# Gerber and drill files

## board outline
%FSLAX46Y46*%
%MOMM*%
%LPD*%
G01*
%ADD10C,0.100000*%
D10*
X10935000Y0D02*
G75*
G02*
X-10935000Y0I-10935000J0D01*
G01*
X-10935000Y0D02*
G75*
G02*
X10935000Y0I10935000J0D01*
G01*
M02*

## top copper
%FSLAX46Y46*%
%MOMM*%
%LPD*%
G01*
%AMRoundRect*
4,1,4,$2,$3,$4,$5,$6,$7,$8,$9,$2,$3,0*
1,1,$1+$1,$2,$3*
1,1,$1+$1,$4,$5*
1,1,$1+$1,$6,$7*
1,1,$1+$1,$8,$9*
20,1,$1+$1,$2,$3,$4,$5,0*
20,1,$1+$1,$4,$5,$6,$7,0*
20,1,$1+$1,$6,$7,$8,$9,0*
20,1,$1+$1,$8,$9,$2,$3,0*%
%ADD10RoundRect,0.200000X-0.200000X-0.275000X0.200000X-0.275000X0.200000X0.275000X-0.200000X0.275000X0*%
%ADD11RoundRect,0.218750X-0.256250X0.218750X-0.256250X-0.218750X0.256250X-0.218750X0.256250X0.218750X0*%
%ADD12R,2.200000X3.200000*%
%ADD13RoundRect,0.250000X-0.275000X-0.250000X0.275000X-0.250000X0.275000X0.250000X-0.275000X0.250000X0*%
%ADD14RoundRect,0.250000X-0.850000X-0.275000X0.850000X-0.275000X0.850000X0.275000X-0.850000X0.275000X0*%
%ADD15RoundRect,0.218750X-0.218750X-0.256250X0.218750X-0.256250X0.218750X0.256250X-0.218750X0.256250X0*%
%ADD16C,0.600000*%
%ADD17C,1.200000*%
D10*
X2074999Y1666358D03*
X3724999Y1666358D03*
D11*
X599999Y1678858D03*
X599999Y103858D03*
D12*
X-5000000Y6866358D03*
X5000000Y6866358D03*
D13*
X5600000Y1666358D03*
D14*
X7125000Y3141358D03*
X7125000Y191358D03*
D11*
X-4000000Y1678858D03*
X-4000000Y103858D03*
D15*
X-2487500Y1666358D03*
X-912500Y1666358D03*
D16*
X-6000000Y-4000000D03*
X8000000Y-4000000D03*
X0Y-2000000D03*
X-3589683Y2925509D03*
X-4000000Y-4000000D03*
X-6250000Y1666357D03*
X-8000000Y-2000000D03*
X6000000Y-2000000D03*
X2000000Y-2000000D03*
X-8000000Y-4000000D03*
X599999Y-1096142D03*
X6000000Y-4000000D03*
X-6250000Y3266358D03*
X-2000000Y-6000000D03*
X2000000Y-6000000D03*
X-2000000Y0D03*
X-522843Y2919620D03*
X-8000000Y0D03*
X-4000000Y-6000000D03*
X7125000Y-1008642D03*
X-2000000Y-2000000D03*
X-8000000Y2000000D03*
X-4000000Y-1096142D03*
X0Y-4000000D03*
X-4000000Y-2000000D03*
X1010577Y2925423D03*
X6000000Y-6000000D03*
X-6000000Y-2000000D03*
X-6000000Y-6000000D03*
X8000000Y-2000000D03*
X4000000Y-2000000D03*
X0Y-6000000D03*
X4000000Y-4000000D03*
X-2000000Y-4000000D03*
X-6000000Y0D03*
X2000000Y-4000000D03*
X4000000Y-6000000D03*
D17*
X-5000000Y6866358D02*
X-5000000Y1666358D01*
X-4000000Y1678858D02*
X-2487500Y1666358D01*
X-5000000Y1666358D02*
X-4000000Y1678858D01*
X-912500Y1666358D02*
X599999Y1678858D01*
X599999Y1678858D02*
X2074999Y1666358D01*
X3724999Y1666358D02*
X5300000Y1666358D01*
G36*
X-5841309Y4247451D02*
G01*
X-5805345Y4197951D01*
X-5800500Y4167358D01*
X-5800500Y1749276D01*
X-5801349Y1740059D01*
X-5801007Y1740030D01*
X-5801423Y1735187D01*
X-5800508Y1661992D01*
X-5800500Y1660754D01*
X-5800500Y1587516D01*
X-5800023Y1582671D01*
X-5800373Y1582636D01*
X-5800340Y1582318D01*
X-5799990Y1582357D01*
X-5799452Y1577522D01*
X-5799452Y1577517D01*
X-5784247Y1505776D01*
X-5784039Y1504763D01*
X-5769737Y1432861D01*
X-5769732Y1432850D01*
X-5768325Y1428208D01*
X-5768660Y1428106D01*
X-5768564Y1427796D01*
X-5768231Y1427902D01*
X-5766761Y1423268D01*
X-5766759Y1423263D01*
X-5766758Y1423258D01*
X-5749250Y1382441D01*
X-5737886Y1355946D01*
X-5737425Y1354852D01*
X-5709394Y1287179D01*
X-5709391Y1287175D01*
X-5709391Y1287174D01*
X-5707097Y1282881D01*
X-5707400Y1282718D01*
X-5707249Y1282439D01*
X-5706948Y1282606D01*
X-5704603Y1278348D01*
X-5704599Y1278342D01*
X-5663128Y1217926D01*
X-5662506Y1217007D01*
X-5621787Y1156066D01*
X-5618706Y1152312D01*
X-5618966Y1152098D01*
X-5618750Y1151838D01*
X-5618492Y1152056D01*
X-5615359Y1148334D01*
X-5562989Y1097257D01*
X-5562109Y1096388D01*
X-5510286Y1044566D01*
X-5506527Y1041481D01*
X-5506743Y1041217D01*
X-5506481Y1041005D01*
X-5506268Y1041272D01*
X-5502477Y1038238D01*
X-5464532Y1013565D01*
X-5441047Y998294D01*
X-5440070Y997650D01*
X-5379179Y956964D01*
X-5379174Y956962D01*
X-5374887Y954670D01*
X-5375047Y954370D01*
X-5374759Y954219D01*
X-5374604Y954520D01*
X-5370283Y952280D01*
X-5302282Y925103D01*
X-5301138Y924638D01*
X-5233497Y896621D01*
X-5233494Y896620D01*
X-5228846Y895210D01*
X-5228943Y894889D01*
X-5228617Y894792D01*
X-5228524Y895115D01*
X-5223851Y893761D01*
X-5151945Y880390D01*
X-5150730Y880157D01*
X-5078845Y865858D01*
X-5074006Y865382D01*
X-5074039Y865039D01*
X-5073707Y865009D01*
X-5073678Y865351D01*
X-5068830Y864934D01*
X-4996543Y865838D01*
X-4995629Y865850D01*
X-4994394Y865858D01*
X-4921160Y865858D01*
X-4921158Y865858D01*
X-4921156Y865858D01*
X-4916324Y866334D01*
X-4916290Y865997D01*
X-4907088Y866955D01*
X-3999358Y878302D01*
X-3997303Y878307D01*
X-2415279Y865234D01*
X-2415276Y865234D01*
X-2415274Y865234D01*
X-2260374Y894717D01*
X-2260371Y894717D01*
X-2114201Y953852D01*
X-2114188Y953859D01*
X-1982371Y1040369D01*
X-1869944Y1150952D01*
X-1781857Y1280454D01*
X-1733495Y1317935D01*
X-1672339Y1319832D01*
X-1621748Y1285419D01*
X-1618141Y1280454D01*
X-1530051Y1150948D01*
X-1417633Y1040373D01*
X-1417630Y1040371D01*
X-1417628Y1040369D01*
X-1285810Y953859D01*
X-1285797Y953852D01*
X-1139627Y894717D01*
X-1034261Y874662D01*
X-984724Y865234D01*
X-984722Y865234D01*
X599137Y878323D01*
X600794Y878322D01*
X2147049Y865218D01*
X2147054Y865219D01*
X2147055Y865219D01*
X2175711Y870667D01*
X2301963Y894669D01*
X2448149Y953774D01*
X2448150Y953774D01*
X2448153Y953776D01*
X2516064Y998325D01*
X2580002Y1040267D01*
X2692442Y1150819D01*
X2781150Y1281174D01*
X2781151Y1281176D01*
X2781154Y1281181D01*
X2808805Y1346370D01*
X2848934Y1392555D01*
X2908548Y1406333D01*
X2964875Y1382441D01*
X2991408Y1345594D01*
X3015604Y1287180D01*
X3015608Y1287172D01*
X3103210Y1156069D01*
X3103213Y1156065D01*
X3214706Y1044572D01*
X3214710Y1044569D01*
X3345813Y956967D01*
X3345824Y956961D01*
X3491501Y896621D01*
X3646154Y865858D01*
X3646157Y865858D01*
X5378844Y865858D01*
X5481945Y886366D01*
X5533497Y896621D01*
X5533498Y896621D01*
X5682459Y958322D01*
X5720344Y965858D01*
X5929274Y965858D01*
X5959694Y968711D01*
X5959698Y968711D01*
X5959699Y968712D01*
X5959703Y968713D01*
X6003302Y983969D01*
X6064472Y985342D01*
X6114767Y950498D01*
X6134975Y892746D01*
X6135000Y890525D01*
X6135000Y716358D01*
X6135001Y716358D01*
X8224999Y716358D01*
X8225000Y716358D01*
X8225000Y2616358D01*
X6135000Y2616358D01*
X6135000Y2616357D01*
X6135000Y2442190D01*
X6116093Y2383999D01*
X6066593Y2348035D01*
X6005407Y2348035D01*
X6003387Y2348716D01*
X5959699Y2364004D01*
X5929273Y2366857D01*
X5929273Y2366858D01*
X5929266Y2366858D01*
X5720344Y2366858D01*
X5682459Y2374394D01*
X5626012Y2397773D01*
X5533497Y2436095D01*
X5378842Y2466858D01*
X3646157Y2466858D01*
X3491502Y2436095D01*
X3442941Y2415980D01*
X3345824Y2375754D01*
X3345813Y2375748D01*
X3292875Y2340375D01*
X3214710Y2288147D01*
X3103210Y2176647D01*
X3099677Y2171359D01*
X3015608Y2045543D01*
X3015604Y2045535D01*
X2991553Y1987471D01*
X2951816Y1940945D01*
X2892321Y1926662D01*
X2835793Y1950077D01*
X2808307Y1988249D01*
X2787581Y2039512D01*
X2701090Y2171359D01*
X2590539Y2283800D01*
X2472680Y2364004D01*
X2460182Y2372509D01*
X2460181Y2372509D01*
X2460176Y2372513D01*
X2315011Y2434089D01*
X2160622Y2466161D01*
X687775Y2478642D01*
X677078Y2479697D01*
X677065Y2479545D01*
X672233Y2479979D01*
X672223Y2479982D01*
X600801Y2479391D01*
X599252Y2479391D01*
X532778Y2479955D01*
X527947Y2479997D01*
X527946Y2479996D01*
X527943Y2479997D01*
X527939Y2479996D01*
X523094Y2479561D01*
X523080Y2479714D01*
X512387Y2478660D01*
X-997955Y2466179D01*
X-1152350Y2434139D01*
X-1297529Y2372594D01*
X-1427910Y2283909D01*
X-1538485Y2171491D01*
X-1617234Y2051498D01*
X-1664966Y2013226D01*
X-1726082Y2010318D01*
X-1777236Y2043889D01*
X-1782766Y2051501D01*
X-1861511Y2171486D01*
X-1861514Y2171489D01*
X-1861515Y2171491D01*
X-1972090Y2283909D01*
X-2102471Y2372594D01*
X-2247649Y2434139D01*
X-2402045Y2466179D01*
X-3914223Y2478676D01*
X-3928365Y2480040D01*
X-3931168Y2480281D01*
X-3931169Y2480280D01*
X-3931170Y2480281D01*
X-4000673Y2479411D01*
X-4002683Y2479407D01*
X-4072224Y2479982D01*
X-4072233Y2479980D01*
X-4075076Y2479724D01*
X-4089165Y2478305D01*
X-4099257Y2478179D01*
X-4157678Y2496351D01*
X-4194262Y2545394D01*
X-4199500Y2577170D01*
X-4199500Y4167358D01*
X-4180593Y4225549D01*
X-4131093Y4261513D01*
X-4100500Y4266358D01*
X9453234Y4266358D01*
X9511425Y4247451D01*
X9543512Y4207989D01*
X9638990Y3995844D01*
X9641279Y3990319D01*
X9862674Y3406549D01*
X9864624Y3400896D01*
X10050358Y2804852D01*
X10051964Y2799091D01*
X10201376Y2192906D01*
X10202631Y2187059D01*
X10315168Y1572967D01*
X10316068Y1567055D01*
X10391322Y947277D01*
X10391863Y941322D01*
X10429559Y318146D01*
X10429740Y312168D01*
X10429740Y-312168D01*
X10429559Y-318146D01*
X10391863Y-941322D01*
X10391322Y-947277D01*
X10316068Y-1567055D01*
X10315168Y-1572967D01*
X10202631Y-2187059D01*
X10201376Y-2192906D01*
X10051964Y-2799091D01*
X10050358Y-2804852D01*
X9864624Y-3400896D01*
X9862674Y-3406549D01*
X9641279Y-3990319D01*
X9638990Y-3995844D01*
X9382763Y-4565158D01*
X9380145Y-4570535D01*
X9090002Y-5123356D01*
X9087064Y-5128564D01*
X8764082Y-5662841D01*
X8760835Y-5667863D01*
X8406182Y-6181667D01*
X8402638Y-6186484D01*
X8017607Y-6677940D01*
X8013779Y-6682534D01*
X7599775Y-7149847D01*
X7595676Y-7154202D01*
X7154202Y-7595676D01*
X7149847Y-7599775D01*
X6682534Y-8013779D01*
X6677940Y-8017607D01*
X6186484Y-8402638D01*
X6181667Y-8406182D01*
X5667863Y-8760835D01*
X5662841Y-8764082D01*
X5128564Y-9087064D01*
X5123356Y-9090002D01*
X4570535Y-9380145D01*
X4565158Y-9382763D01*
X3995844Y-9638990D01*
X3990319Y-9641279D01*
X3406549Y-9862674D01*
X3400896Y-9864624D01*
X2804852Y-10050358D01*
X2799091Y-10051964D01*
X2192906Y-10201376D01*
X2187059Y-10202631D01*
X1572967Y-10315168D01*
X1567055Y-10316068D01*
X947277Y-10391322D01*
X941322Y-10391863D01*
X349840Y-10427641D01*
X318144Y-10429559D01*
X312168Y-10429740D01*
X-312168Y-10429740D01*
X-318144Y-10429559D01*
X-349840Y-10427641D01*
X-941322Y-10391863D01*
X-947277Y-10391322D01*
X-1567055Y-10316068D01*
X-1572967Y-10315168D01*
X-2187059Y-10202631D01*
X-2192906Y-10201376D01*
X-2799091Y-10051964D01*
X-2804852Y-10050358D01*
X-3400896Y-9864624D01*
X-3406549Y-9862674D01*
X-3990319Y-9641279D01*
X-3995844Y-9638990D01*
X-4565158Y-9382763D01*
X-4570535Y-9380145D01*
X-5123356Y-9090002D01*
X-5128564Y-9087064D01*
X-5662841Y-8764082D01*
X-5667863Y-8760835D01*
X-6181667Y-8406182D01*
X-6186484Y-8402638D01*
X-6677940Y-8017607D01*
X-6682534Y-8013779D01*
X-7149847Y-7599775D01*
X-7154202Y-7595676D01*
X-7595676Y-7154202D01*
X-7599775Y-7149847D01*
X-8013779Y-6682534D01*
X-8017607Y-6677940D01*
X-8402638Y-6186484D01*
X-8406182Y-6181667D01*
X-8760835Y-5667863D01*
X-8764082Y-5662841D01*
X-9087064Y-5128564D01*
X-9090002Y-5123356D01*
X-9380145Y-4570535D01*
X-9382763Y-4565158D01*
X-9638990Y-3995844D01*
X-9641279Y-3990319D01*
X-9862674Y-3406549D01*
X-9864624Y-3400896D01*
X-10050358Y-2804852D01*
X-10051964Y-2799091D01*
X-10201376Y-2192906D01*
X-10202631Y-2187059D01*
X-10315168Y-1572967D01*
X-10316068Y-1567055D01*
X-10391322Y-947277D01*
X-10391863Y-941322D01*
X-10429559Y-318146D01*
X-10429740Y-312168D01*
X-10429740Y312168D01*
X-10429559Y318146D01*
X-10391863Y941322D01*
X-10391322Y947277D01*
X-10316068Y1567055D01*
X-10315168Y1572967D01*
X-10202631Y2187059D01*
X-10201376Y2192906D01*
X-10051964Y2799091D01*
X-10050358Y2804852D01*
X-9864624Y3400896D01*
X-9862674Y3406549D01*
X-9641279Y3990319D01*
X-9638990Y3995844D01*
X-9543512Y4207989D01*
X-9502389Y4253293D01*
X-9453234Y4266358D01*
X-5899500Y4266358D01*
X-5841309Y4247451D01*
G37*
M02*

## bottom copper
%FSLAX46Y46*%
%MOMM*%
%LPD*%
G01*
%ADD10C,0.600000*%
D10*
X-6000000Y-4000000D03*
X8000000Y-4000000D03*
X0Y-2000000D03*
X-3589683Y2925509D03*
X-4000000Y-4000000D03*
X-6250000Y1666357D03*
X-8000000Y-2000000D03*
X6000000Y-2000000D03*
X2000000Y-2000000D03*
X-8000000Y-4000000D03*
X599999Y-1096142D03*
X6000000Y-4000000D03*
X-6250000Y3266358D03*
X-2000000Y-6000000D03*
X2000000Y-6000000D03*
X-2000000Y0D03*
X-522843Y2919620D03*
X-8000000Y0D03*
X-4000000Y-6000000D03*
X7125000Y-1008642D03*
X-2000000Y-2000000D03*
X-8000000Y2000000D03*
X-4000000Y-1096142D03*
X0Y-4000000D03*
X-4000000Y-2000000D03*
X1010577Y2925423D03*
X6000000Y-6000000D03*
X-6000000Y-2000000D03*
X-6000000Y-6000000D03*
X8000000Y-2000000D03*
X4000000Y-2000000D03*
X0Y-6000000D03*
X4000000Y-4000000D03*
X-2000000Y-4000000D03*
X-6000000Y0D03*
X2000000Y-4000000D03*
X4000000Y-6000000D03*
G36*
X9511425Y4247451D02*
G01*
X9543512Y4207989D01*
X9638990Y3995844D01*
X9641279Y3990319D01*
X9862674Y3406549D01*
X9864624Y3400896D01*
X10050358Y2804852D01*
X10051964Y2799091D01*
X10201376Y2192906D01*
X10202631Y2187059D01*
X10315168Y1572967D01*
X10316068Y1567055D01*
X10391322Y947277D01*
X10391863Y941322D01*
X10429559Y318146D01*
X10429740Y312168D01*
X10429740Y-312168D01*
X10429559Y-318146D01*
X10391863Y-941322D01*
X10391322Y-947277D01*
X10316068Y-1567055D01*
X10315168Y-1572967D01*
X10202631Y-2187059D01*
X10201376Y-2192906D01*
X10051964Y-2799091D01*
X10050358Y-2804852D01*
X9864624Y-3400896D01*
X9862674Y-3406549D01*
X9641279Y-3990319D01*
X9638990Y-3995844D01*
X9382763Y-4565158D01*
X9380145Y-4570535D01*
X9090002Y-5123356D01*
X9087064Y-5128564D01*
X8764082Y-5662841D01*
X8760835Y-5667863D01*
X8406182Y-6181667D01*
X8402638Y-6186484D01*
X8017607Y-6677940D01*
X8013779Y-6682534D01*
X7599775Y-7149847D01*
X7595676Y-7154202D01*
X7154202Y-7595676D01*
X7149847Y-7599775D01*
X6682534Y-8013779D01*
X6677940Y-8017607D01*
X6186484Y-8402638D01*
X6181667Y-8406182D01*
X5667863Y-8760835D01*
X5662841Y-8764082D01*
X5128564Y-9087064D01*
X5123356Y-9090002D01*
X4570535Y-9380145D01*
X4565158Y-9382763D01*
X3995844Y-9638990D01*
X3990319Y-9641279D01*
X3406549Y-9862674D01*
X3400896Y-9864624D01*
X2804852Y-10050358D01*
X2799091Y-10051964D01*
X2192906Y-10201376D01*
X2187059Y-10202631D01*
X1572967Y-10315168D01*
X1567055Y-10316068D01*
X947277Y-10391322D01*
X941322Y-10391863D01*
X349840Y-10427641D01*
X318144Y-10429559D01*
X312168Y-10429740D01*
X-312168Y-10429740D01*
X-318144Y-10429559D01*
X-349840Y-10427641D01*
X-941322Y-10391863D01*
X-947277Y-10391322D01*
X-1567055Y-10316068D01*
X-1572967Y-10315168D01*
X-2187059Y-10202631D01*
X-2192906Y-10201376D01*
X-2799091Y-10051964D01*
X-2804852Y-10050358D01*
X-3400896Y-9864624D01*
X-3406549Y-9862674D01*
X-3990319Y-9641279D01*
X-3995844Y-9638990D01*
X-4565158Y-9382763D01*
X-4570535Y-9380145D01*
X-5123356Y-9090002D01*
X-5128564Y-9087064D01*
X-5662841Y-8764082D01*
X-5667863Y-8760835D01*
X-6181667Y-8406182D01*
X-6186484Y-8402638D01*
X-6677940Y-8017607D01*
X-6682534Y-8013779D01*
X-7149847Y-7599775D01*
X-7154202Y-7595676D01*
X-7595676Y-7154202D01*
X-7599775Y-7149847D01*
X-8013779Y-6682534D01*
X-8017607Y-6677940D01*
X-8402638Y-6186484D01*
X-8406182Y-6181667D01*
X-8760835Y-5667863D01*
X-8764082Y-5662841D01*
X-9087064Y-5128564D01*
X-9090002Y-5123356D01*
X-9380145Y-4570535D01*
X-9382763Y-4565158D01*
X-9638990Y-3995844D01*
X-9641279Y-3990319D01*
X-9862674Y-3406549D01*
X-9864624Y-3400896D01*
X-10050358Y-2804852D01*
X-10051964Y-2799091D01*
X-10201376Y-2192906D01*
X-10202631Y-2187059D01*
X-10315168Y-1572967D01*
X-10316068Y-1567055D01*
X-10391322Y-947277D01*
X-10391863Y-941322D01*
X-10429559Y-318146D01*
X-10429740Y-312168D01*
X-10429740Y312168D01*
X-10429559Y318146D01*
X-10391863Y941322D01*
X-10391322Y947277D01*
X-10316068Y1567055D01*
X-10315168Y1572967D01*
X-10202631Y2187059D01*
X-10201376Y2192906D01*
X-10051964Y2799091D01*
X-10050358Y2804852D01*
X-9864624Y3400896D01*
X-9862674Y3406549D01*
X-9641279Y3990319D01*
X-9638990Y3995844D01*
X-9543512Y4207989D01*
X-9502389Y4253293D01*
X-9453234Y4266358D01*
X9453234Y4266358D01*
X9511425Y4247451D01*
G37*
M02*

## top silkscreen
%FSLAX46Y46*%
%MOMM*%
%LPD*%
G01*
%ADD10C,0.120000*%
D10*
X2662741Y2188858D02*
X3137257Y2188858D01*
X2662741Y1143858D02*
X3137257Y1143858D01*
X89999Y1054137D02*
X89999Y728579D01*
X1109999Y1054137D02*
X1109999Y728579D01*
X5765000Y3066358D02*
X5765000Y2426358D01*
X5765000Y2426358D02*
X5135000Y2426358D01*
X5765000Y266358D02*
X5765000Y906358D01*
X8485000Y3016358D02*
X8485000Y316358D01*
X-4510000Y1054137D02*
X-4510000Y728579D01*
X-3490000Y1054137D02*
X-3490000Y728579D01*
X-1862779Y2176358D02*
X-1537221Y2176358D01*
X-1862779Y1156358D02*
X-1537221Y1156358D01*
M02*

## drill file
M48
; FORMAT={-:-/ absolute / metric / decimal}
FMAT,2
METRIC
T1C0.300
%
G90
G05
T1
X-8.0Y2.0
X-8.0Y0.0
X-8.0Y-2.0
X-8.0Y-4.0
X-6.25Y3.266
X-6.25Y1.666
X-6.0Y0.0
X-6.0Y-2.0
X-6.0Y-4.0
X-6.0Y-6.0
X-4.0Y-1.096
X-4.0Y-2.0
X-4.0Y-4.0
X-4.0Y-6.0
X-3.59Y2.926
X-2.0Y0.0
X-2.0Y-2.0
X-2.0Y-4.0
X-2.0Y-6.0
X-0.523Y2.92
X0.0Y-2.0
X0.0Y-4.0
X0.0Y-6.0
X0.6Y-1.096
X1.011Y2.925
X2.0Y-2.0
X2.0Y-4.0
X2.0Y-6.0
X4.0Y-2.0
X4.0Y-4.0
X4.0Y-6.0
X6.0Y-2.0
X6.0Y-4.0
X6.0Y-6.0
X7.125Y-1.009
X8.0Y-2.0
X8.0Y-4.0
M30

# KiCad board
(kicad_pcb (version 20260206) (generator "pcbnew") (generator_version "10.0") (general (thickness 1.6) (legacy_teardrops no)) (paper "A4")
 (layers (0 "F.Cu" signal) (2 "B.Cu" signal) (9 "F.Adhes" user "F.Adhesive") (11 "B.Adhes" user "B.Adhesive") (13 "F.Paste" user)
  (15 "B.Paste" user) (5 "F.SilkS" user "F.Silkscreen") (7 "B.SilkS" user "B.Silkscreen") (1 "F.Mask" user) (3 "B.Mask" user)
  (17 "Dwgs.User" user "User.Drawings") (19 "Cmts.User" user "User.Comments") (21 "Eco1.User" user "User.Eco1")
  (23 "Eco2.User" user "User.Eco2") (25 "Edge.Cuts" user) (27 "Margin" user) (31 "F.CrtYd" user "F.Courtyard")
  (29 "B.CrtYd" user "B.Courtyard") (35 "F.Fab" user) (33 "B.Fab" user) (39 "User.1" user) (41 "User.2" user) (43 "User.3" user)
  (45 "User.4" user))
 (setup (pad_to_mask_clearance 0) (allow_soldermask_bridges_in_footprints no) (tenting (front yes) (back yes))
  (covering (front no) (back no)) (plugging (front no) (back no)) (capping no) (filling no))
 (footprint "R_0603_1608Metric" (layer "F.Cu") (at 2.899999 -1.666358)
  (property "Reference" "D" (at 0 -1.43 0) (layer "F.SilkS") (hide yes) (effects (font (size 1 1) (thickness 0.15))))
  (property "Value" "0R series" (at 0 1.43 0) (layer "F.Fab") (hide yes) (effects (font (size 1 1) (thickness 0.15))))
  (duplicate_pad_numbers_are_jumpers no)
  (fp_line (start -0.237258 -0.5225) (end 0.237258 -0.5225) (stroke (width 0.12) (type solid)) (layer "F.SilkS"))
  (fp_line (start -0.237258 0.5225) (end 0.237258 0.5225) (stroke (width 0.12) (type solid)) (layer "F.SilkS"))
  (pad "1" smd roundrect (at -0.825 0) (size 0.8 0.95) (layers "F.Cu" "F.Mask" "F.Paste") (roundrect_rratio 0.25) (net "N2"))
  (pad "2" smd roundrect (at 0.825 0) (size 0.8 0.95) (layers "F.Cu" "F.Mask" "F.Paste") (roundrect_rratio 0.25) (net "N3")))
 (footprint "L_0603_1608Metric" (layer "F.Cu") (at 0.599999 -0.891358 -90)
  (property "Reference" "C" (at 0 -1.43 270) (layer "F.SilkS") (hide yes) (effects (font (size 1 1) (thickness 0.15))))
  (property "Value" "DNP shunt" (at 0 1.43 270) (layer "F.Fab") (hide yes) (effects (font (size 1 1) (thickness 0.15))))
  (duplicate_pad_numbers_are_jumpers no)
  (fp_line (start -0.162779 0.51) (end 0.162779 0.51) (stroke (width 0.12) (type solid)) (layer "F.SilkS"))
  (fp_line (start -0.162779 -0.51) (end 0.162779 -0.51) (stroke (width 0.12) (type solid)) (layer "F.SilkS"))
  (pad "1" smd roundrect (at -0.7875 0 270) (size 0.875 0.95) (layers "F.Cu" "F.Mask" "F.Paste") (roundrect_rratio 0.25) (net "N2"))
  (pad "2" smd roundrect (at 0.7875 0 270) (size 0.875 0.95) (layers "F.Cu" "F.Mask" "F.Paste") (roundrect_rratio 0.25) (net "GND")))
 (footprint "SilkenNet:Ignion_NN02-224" (layer "F.Cu") (at 0 -6.866358)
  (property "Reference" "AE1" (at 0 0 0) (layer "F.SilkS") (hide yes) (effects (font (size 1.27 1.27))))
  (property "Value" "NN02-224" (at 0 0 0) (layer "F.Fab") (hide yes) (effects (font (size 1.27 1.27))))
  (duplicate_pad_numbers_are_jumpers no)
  (pad "1" smd rect (at -5 0) (size 2.2 3.2) (layers "F.Cu" "F.Mask" "F.Paste") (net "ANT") (thermal_bridge_angle 45))
  (pad "2" smd rect (at 5 0) (size 2.2 3.2) (layers "F.Cu" "F.Mask" "F.Paste") (thermal_bridge_angle 45)))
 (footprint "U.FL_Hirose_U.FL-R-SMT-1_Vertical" (layer "F.Cu") (at 7.125 -1.666358)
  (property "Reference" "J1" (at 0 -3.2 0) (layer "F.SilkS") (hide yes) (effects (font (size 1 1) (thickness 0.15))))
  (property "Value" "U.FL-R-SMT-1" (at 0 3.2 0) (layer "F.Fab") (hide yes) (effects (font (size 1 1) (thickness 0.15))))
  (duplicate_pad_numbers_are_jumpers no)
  (fp_line (start -1.36 -1.4) (end -1.36 -0.76) (stroke (width 0.12) (type solid)) (layer "F.SilkS"))
  (fp_line (start -1.36 -0.76) (end -1.99 -0.76) (stroke (width 0.12) (type solid)) (layer "F.SilkS"))
  (fp_line (start -1.36 1.4) (end -1.36 0.76) (stroke (width 0.12) (type solid)) (layer "F.SilkS"))
  (fp_line (start 1.36 -1.35) (end 1.36 1.35) (stroke (width 0.12) (type solid)) (layer "F.SilkS"))
  (pad "1" smd roundrect (at -1.525 0) (size 1.05 1) (layers "F.Cu" "F.Mask" "F.Paste") (roundrect_rratio 0.25) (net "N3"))
  (pad "2" smd roundrect (at 0 -1.475) (size 2.2 1.05) (layers "F.Cu" "F.Mask" "F.Paste") (roundrect_rratio 0.2380952381) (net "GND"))
  (pad "2" smd roundrect (at 0 1.475) (size 2.2 1.05) (layers "F.Cu" "F.Mask" "F.Paste") (roundrect_rratio 0.2380952381) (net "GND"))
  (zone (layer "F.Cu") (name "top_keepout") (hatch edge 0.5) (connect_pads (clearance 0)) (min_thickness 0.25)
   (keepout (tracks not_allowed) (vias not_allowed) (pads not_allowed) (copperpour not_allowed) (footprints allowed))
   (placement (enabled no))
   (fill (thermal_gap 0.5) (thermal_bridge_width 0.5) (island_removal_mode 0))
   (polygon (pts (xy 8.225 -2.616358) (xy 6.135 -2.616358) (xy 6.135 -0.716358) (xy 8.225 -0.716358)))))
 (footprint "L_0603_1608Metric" (layer "F.Cu") (at -4 -0.891358 -90)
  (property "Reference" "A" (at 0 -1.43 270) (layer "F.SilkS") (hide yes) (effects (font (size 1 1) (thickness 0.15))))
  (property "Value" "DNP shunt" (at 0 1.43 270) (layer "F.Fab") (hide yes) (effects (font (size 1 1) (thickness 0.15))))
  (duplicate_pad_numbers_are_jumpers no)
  (fp_line (start -0.162779 0.51) (end 0.162779 0.51) (stroke (width 0.12) (type solid)) (layer "F.SilkS"))
  (fp_line (start -0.162779 -0.51) (end 0.162779 -0.51) (stroke (width 0.12) (type solid)) (layer "F.SilkS"))
  (pad "1" smd roundrect (at -0.7875 0 270) (size 0.875 0.95) (layers "F.Cu" "F.Mask" "F.Paste") (roundrect_rratio 0.25) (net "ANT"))
  (pad "2" smd roundrect (at 0.7875 0 270) (size 0.875 0.95) (layers "F.Cu" "F.Mask" "F.Paste") (roundrect_rratio 0.25) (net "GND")))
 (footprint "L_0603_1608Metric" (layer "F.Cu") (at -1.7 -1.666358)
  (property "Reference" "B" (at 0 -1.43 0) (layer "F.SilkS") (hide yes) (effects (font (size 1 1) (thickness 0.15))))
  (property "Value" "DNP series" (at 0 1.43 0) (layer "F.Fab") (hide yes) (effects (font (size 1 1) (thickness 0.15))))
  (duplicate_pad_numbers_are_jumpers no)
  (fp_line (start -0.162779 -0.51) (end 0.162779 -0.51) (stroke (width 0.12) (type solid)) (layer "F.SilkS"))
  (fp_line (start -0.162779 0.51) (end 0.162779 0.51) (stroke (width 0.12) (type solid)) (layer "F.SilkS"))
  (pad "1" smd roundrect (at -0.7875 0) (size 0.875 0.95) (layers "F.Cu" "F.Mask" "F.Paste") (roundrect_rratio 0.25) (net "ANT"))
  (pad "2" smd roundrect (at 0.7875 0) (size 0.875 0.95) (layers "F.Cu" "F.Mask" "F.Paste") (roundrect_rratio 0.25) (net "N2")))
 (gr_circle (center 0 0) (end 10.935 0) (stroke (width 0.1) (type default)) (fill no) (layer "Edge.Cuts"))
 (via (at -6 4) (size 0.6) (drill 0.3) (layers "F.Cu" "B.Cu") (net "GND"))
 (via (at 8 4) (size 0.6) (drill 0.3) (layers "F.Cu" "B.Cu") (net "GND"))
 (via (at 0 2) (size 0.6) (drill 0.3) (layers "F.Cu" "B.Cu") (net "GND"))
 (via (at -3.589683 -2.925509) (size 0.6) (drill 0.3) (layers "F.Cu" "B.Cu") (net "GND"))
 (via (at -4 4) (size 0.6) (drill 0.3) (layers "F.Cu" "B.Cu") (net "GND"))
 (via (at -6.25 -1.666357) (size 0.6) (drill 0.3) (layers "F.Cu" "B.Cu") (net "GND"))
 (via (at -8 2) (size 0.6) (drill 0.3) (layers "F.Cu" "B.Cu") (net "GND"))
 (via (at 6 2) (size 0.6) (drill 0.3) (layers "F.Cu" "B.Cu") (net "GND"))
 (via (at 2 2) (size 0.6) (drill 0.3) (layers "F.Cu" "B.Cu") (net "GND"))
 (via (at -8 4) (size 0.6) (drill 0.3) (layers "F.Cu" "B.Cu") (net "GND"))
 (via (at 0.599999 1.096142) (size 0.6) (drill 0.3) (layers "F.Cu" "B.Cu") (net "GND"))
 (via (at 6 4) (size 0.6) (drill 0.3) (layers "F.Cu" "B.Cu") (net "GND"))
 (via (at -6.25 -3.266358) (size 0.6) (drill 0.3) (layers "F.Cu" "B.Cu") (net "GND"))
 (via (at -2 6) (size 0.6) (drill 0.3) (layers "F.Cu" "B.Cu") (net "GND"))
 (via (at 2 6) (size 0.6) (drill 0.3) (layers "F.Cu" "B.Cu") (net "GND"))
 (via (at -2 0) (size 0.6) (drill 0.3) (layers "F.Cu" "B.Cu") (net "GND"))
 (via (at -0.522843 -2.91962) (size 0.6) (drill 0.3) (layers "F.Cu" "B.Cu") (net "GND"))
 (via (at -8 0) (size 0.6) (drill 0.3) (layers "F.Cu" "B.Cu") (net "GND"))
 (via (at -4 6) (size 0.6) (drill 0.3) (layers "F.Cu" "B.Cu") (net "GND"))
 (via (at 7.125 1.008642) (size 0.6) (drill 0.3) (layers "F.Cu" "B.Cu") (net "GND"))
 (via (at -2 2) (size 0.6) (drill 0.3) (layers "F.Cu" "B.Cu") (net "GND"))
 (via (at -8 -2) (size 0.6) (drill 0.3) (layers "F.Cu" "B.Cu") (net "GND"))
 (via (at -4 1.096142) (size 0.6) (drill 0.3) (layers "F.Cu" "B.Cu") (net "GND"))
 (via (at 0 4) (size 0.6) (drill 0.3) (layers "F.Cu" "B.Cu") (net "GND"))
 (via (at -4 2) (size 0.6) (drill 0.3) (layers "F.Cu" "B.Cu") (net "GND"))
 (via (at 1.010577 -2.925423) (size 0.6) (drill 0.3) (layers "F.Cu" "B.Cu") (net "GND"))
 (via (at 6 6) (size 0.6) (drill 0.3) (layers "F.Cu" "B.Cu") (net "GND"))
 (via (at -6 2) (size 0.6) (drill 0.3) (layers "F.Cu" "B.Cu") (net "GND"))
 (via (at -6 6) (size 0.6) (drill 0.3) (layers "F.Cu" "B.Cu") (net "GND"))
 (via (at 8 2) (size 0.6) (drill 0.3) (layers "F.Cu" "B.Cu") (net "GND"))
 (via (at 4 2) (size 0.6) (drill 0.3) (layers "F.Cu" "B.Cu") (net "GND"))
 (via (at 0 6) (size 0.6) (drill 0.3) (layers "F.Cu" "B.Cu") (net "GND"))
 (via (at 4 4) (size 0.6) (drill 0.3) (layers "F.Cu" "B.Cu") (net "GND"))
 (via (at -2 4) (size 0.6) (drill 0.3) (layers "F.Cu" "B.Cu") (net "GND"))
 (via (at -6 0) (size 0.6) (drill 0.3) (layers "F.Cu" "B.Cu") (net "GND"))
 (via (at 2 4) (size 0.6) (drill 0.3) (layers "F.Cu" "B.Cu") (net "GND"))
 (via (at 4 6) (size 0.6) (drill 0.3) (layers "F.Cu" "B.Cu") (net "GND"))
 (segment (start -5 -6.866358) (end -5 -1.666358) (width 1.2) (layer "F.Cu") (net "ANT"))
 (segment (start -4 -1.678858) (end -2.4875 -1.666358) (width 1.2) (layer "F.Cu") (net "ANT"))
 (segment (start -5 -1.666358) (end -4 -1.678858) (width 1.2) (layer "F.Cu") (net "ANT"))
 (segment (start -0.9125 -1.666358) (end 0.599999 -1.678858) (width 1.2) (layer "F.Cu") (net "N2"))
 (segment (start 0.599999 -1.678858) (end 2.074999 -1.666358) (width 1.2) (layer "F.Cu") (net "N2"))
 (segment (start 3.724999 -1.666358) (end 5.3 -1.666358) (width 1.2) (layer "F.Cu") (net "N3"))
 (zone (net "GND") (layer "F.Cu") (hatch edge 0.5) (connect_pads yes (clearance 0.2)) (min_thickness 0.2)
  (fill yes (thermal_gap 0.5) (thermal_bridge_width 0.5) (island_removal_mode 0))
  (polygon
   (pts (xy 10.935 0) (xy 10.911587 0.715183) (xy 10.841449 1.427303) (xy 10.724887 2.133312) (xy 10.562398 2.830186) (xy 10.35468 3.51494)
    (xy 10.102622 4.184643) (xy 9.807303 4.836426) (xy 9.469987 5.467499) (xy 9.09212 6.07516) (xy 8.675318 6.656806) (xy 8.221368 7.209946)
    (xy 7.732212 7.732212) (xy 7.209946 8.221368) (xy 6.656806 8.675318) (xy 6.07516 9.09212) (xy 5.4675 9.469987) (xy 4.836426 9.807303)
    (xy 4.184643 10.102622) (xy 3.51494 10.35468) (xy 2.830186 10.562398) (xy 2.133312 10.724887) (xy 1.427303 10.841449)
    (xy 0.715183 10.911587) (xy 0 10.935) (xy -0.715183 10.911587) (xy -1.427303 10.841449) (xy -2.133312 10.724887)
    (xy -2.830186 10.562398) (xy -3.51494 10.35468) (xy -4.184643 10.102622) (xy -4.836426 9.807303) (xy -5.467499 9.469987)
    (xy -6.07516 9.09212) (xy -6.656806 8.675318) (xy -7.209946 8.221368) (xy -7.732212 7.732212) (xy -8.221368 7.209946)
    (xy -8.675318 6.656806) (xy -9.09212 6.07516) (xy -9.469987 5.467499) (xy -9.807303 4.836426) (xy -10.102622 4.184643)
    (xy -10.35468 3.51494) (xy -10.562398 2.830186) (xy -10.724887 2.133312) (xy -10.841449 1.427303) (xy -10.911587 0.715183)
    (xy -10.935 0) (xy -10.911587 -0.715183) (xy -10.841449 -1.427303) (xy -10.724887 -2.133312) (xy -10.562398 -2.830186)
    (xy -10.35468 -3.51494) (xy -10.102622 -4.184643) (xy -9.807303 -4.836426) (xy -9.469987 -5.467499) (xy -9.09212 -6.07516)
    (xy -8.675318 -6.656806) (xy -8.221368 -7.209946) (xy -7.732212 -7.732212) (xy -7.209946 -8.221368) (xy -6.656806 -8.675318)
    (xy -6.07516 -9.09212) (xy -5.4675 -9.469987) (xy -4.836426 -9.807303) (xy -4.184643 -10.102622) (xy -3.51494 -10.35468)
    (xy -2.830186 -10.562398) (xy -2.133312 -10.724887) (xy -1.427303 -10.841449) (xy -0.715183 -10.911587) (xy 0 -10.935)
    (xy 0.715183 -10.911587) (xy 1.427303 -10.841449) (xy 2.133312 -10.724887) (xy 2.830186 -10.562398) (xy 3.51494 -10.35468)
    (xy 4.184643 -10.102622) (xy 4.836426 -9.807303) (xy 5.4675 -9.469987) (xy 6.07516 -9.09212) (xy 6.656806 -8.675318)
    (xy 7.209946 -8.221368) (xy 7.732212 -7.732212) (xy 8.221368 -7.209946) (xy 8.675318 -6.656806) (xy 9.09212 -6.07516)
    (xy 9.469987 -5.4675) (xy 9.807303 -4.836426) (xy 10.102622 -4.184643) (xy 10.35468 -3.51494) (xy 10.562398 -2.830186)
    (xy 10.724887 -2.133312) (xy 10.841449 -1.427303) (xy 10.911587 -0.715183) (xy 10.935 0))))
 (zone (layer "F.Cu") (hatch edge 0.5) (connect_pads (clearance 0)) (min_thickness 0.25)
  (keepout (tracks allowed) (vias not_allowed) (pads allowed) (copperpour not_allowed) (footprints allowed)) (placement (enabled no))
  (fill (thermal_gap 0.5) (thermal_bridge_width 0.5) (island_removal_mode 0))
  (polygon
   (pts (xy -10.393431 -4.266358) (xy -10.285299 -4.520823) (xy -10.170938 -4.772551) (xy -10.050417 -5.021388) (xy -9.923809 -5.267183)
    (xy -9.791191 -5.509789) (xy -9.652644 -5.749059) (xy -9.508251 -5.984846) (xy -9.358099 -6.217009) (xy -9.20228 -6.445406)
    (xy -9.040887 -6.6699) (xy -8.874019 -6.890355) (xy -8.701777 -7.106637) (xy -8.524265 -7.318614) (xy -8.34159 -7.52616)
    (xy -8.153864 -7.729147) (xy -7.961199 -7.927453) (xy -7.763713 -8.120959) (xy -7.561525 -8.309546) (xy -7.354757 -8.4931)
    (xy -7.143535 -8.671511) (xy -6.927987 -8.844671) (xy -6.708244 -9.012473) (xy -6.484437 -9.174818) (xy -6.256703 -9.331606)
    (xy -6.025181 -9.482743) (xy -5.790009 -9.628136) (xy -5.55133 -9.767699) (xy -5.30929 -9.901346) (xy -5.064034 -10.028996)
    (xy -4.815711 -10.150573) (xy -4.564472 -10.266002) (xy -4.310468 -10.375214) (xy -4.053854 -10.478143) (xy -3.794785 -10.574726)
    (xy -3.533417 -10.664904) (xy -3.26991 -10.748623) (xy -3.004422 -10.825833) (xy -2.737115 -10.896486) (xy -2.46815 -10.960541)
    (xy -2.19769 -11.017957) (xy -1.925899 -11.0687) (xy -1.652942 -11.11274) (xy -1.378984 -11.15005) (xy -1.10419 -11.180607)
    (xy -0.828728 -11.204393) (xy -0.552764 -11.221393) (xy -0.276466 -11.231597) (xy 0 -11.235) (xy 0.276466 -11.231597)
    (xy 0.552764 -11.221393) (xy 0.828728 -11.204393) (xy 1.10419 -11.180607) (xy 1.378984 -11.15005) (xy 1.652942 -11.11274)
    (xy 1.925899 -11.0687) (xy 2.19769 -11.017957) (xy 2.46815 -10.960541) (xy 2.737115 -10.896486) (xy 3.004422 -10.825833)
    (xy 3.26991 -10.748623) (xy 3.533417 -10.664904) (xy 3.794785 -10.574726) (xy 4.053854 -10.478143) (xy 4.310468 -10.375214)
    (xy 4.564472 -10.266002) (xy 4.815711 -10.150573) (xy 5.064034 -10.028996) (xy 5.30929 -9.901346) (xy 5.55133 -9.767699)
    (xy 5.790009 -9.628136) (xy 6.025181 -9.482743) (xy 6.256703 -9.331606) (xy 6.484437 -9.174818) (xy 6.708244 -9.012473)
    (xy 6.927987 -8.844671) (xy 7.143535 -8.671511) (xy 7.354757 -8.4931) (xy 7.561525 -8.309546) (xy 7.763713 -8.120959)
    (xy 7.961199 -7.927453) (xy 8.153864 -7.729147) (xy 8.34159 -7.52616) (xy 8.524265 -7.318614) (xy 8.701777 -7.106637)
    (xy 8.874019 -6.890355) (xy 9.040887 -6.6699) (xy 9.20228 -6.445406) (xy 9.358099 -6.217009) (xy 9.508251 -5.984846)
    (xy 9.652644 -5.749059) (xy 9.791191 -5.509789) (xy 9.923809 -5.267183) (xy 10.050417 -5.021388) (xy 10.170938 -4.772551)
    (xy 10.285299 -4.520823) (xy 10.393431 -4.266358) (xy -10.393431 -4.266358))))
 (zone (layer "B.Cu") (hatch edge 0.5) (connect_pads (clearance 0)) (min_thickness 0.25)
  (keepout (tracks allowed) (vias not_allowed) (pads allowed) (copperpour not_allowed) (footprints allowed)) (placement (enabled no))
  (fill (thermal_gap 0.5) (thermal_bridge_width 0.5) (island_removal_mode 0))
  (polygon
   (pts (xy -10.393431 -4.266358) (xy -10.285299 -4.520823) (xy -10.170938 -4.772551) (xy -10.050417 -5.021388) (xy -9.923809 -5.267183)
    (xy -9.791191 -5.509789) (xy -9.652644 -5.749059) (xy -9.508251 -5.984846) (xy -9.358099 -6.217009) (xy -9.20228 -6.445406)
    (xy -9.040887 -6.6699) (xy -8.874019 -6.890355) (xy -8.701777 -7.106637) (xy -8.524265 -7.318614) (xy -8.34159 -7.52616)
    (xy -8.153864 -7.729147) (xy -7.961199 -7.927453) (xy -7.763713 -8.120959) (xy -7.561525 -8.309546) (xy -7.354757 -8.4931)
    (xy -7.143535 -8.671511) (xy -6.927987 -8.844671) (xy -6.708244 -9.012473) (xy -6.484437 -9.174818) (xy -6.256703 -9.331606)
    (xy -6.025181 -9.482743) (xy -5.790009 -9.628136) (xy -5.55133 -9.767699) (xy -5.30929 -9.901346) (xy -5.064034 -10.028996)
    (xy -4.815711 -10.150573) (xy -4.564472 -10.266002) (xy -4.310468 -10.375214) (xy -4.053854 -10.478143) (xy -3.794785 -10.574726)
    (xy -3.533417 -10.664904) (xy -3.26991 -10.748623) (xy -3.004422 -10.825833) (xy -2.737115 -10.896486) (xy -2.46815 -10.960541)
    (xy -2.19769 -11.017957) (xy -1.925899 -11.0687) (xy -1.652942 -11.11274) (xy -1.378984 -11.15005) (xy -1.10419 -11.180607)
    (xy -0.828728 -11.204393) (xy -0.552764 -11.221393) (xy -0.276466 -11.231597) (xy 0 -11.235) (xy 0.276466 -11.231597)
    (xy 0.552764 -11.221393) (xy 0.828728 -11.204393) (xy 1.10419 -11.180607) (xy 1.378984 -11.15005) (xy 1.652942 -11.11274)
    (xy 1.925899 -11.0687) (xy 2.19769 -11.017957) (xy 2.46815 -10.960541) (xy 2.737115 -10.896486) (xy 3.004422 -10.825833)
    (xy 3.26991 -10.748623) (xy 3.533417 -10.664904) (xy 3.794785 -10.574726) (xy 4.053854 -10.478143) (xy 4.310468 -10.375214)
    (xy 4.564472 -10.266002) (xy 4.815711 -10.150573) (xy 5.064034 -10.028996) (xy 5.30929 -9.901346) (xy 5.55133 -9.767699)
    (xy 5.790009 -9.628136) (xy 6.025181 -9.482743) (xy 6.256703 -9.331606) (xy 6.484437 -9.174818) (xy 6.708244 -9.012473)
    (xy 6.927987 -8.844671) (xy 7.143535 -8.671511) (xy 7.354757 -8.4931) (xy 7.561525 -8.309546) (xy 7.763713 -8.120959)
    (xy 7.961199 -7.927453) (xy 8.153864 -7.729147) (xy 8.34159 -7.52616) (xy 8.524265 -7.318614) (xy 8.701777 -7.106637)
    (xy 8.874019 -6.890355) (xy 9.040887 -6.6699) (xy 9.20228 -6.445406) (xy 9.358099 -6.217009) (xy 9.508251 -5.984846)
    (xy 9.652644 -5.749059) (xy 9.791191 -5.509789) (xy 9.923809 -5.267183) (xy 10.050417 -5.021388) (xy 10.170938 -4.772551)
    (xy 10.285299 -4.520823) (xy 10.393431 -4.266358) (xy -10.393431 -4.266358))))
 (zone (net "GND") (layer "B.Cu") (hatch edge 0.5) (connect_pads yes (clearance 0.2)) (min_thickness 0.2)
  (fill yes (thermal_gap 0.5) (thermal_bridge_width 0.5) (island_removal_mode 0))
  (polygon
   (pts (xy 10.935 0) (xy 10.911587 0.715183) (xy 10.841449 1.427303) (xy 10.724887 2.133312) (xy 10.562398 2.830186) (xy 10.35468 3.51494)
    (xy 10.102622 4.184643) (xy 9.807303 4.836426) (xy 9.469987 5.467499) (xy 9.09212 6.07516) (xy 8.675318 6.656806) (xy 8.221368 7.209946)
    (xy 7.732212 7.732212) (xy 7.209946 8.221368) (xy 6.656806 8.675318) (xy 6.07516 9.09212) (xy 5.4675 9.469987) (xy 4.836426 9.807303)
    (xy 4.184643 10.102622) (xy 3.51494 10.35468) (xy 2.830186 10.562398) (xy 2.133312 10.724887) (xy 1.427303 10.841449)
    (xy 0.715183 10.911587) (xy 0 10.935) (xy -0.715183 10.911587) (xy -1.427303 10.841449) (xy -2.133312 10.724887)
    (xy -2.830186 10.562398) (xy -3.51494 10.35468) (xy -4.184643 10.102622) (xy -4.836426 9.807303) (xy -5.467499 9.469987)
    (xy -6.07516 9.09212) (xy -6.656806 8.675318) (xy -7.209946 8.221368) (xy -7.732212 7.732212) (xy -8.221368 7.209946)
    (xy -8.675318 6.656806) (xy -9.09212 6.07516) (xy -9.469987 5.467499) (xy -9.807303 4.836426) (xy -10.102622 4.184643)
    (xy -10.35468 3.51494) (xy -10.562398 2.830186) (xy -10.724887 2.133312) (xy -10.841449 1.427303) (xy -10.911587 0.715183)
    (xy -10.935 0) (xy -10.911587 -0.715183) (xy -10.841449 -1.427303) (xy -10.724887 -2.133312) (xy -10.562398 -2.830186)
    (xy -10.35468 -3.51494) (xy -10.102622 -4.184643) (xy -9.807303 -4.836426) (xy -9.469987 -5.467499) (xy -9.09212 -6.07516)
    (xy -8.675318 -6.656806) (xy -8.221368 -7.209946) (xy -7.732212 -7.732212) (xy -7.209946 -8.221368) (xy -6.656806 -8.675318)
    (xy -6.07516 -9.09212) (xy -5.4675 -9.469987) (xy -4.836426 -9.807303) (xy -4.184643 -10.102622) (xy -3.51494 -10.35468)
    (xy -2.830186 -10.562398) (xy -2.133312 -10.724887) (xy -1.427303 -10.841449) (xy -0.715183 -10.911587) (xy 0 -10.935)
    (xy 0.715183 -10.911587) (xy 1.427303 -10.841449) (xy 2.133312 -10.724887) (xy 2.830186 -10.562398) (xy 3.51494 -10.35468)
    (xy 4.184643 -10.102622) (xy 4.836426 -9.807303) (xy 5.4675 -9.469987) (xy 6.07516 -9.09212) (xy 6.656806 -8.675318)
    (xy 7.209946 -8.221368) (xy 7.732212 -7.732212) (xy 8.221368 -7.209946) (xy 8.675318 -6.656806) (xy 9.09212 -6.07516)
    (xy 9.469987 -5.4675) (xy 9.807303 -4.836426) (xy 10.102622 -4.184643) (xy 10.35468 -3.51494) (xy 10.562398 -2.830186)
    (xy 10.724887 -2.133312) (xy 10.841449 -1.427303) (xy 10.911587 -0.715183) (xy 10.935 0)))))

